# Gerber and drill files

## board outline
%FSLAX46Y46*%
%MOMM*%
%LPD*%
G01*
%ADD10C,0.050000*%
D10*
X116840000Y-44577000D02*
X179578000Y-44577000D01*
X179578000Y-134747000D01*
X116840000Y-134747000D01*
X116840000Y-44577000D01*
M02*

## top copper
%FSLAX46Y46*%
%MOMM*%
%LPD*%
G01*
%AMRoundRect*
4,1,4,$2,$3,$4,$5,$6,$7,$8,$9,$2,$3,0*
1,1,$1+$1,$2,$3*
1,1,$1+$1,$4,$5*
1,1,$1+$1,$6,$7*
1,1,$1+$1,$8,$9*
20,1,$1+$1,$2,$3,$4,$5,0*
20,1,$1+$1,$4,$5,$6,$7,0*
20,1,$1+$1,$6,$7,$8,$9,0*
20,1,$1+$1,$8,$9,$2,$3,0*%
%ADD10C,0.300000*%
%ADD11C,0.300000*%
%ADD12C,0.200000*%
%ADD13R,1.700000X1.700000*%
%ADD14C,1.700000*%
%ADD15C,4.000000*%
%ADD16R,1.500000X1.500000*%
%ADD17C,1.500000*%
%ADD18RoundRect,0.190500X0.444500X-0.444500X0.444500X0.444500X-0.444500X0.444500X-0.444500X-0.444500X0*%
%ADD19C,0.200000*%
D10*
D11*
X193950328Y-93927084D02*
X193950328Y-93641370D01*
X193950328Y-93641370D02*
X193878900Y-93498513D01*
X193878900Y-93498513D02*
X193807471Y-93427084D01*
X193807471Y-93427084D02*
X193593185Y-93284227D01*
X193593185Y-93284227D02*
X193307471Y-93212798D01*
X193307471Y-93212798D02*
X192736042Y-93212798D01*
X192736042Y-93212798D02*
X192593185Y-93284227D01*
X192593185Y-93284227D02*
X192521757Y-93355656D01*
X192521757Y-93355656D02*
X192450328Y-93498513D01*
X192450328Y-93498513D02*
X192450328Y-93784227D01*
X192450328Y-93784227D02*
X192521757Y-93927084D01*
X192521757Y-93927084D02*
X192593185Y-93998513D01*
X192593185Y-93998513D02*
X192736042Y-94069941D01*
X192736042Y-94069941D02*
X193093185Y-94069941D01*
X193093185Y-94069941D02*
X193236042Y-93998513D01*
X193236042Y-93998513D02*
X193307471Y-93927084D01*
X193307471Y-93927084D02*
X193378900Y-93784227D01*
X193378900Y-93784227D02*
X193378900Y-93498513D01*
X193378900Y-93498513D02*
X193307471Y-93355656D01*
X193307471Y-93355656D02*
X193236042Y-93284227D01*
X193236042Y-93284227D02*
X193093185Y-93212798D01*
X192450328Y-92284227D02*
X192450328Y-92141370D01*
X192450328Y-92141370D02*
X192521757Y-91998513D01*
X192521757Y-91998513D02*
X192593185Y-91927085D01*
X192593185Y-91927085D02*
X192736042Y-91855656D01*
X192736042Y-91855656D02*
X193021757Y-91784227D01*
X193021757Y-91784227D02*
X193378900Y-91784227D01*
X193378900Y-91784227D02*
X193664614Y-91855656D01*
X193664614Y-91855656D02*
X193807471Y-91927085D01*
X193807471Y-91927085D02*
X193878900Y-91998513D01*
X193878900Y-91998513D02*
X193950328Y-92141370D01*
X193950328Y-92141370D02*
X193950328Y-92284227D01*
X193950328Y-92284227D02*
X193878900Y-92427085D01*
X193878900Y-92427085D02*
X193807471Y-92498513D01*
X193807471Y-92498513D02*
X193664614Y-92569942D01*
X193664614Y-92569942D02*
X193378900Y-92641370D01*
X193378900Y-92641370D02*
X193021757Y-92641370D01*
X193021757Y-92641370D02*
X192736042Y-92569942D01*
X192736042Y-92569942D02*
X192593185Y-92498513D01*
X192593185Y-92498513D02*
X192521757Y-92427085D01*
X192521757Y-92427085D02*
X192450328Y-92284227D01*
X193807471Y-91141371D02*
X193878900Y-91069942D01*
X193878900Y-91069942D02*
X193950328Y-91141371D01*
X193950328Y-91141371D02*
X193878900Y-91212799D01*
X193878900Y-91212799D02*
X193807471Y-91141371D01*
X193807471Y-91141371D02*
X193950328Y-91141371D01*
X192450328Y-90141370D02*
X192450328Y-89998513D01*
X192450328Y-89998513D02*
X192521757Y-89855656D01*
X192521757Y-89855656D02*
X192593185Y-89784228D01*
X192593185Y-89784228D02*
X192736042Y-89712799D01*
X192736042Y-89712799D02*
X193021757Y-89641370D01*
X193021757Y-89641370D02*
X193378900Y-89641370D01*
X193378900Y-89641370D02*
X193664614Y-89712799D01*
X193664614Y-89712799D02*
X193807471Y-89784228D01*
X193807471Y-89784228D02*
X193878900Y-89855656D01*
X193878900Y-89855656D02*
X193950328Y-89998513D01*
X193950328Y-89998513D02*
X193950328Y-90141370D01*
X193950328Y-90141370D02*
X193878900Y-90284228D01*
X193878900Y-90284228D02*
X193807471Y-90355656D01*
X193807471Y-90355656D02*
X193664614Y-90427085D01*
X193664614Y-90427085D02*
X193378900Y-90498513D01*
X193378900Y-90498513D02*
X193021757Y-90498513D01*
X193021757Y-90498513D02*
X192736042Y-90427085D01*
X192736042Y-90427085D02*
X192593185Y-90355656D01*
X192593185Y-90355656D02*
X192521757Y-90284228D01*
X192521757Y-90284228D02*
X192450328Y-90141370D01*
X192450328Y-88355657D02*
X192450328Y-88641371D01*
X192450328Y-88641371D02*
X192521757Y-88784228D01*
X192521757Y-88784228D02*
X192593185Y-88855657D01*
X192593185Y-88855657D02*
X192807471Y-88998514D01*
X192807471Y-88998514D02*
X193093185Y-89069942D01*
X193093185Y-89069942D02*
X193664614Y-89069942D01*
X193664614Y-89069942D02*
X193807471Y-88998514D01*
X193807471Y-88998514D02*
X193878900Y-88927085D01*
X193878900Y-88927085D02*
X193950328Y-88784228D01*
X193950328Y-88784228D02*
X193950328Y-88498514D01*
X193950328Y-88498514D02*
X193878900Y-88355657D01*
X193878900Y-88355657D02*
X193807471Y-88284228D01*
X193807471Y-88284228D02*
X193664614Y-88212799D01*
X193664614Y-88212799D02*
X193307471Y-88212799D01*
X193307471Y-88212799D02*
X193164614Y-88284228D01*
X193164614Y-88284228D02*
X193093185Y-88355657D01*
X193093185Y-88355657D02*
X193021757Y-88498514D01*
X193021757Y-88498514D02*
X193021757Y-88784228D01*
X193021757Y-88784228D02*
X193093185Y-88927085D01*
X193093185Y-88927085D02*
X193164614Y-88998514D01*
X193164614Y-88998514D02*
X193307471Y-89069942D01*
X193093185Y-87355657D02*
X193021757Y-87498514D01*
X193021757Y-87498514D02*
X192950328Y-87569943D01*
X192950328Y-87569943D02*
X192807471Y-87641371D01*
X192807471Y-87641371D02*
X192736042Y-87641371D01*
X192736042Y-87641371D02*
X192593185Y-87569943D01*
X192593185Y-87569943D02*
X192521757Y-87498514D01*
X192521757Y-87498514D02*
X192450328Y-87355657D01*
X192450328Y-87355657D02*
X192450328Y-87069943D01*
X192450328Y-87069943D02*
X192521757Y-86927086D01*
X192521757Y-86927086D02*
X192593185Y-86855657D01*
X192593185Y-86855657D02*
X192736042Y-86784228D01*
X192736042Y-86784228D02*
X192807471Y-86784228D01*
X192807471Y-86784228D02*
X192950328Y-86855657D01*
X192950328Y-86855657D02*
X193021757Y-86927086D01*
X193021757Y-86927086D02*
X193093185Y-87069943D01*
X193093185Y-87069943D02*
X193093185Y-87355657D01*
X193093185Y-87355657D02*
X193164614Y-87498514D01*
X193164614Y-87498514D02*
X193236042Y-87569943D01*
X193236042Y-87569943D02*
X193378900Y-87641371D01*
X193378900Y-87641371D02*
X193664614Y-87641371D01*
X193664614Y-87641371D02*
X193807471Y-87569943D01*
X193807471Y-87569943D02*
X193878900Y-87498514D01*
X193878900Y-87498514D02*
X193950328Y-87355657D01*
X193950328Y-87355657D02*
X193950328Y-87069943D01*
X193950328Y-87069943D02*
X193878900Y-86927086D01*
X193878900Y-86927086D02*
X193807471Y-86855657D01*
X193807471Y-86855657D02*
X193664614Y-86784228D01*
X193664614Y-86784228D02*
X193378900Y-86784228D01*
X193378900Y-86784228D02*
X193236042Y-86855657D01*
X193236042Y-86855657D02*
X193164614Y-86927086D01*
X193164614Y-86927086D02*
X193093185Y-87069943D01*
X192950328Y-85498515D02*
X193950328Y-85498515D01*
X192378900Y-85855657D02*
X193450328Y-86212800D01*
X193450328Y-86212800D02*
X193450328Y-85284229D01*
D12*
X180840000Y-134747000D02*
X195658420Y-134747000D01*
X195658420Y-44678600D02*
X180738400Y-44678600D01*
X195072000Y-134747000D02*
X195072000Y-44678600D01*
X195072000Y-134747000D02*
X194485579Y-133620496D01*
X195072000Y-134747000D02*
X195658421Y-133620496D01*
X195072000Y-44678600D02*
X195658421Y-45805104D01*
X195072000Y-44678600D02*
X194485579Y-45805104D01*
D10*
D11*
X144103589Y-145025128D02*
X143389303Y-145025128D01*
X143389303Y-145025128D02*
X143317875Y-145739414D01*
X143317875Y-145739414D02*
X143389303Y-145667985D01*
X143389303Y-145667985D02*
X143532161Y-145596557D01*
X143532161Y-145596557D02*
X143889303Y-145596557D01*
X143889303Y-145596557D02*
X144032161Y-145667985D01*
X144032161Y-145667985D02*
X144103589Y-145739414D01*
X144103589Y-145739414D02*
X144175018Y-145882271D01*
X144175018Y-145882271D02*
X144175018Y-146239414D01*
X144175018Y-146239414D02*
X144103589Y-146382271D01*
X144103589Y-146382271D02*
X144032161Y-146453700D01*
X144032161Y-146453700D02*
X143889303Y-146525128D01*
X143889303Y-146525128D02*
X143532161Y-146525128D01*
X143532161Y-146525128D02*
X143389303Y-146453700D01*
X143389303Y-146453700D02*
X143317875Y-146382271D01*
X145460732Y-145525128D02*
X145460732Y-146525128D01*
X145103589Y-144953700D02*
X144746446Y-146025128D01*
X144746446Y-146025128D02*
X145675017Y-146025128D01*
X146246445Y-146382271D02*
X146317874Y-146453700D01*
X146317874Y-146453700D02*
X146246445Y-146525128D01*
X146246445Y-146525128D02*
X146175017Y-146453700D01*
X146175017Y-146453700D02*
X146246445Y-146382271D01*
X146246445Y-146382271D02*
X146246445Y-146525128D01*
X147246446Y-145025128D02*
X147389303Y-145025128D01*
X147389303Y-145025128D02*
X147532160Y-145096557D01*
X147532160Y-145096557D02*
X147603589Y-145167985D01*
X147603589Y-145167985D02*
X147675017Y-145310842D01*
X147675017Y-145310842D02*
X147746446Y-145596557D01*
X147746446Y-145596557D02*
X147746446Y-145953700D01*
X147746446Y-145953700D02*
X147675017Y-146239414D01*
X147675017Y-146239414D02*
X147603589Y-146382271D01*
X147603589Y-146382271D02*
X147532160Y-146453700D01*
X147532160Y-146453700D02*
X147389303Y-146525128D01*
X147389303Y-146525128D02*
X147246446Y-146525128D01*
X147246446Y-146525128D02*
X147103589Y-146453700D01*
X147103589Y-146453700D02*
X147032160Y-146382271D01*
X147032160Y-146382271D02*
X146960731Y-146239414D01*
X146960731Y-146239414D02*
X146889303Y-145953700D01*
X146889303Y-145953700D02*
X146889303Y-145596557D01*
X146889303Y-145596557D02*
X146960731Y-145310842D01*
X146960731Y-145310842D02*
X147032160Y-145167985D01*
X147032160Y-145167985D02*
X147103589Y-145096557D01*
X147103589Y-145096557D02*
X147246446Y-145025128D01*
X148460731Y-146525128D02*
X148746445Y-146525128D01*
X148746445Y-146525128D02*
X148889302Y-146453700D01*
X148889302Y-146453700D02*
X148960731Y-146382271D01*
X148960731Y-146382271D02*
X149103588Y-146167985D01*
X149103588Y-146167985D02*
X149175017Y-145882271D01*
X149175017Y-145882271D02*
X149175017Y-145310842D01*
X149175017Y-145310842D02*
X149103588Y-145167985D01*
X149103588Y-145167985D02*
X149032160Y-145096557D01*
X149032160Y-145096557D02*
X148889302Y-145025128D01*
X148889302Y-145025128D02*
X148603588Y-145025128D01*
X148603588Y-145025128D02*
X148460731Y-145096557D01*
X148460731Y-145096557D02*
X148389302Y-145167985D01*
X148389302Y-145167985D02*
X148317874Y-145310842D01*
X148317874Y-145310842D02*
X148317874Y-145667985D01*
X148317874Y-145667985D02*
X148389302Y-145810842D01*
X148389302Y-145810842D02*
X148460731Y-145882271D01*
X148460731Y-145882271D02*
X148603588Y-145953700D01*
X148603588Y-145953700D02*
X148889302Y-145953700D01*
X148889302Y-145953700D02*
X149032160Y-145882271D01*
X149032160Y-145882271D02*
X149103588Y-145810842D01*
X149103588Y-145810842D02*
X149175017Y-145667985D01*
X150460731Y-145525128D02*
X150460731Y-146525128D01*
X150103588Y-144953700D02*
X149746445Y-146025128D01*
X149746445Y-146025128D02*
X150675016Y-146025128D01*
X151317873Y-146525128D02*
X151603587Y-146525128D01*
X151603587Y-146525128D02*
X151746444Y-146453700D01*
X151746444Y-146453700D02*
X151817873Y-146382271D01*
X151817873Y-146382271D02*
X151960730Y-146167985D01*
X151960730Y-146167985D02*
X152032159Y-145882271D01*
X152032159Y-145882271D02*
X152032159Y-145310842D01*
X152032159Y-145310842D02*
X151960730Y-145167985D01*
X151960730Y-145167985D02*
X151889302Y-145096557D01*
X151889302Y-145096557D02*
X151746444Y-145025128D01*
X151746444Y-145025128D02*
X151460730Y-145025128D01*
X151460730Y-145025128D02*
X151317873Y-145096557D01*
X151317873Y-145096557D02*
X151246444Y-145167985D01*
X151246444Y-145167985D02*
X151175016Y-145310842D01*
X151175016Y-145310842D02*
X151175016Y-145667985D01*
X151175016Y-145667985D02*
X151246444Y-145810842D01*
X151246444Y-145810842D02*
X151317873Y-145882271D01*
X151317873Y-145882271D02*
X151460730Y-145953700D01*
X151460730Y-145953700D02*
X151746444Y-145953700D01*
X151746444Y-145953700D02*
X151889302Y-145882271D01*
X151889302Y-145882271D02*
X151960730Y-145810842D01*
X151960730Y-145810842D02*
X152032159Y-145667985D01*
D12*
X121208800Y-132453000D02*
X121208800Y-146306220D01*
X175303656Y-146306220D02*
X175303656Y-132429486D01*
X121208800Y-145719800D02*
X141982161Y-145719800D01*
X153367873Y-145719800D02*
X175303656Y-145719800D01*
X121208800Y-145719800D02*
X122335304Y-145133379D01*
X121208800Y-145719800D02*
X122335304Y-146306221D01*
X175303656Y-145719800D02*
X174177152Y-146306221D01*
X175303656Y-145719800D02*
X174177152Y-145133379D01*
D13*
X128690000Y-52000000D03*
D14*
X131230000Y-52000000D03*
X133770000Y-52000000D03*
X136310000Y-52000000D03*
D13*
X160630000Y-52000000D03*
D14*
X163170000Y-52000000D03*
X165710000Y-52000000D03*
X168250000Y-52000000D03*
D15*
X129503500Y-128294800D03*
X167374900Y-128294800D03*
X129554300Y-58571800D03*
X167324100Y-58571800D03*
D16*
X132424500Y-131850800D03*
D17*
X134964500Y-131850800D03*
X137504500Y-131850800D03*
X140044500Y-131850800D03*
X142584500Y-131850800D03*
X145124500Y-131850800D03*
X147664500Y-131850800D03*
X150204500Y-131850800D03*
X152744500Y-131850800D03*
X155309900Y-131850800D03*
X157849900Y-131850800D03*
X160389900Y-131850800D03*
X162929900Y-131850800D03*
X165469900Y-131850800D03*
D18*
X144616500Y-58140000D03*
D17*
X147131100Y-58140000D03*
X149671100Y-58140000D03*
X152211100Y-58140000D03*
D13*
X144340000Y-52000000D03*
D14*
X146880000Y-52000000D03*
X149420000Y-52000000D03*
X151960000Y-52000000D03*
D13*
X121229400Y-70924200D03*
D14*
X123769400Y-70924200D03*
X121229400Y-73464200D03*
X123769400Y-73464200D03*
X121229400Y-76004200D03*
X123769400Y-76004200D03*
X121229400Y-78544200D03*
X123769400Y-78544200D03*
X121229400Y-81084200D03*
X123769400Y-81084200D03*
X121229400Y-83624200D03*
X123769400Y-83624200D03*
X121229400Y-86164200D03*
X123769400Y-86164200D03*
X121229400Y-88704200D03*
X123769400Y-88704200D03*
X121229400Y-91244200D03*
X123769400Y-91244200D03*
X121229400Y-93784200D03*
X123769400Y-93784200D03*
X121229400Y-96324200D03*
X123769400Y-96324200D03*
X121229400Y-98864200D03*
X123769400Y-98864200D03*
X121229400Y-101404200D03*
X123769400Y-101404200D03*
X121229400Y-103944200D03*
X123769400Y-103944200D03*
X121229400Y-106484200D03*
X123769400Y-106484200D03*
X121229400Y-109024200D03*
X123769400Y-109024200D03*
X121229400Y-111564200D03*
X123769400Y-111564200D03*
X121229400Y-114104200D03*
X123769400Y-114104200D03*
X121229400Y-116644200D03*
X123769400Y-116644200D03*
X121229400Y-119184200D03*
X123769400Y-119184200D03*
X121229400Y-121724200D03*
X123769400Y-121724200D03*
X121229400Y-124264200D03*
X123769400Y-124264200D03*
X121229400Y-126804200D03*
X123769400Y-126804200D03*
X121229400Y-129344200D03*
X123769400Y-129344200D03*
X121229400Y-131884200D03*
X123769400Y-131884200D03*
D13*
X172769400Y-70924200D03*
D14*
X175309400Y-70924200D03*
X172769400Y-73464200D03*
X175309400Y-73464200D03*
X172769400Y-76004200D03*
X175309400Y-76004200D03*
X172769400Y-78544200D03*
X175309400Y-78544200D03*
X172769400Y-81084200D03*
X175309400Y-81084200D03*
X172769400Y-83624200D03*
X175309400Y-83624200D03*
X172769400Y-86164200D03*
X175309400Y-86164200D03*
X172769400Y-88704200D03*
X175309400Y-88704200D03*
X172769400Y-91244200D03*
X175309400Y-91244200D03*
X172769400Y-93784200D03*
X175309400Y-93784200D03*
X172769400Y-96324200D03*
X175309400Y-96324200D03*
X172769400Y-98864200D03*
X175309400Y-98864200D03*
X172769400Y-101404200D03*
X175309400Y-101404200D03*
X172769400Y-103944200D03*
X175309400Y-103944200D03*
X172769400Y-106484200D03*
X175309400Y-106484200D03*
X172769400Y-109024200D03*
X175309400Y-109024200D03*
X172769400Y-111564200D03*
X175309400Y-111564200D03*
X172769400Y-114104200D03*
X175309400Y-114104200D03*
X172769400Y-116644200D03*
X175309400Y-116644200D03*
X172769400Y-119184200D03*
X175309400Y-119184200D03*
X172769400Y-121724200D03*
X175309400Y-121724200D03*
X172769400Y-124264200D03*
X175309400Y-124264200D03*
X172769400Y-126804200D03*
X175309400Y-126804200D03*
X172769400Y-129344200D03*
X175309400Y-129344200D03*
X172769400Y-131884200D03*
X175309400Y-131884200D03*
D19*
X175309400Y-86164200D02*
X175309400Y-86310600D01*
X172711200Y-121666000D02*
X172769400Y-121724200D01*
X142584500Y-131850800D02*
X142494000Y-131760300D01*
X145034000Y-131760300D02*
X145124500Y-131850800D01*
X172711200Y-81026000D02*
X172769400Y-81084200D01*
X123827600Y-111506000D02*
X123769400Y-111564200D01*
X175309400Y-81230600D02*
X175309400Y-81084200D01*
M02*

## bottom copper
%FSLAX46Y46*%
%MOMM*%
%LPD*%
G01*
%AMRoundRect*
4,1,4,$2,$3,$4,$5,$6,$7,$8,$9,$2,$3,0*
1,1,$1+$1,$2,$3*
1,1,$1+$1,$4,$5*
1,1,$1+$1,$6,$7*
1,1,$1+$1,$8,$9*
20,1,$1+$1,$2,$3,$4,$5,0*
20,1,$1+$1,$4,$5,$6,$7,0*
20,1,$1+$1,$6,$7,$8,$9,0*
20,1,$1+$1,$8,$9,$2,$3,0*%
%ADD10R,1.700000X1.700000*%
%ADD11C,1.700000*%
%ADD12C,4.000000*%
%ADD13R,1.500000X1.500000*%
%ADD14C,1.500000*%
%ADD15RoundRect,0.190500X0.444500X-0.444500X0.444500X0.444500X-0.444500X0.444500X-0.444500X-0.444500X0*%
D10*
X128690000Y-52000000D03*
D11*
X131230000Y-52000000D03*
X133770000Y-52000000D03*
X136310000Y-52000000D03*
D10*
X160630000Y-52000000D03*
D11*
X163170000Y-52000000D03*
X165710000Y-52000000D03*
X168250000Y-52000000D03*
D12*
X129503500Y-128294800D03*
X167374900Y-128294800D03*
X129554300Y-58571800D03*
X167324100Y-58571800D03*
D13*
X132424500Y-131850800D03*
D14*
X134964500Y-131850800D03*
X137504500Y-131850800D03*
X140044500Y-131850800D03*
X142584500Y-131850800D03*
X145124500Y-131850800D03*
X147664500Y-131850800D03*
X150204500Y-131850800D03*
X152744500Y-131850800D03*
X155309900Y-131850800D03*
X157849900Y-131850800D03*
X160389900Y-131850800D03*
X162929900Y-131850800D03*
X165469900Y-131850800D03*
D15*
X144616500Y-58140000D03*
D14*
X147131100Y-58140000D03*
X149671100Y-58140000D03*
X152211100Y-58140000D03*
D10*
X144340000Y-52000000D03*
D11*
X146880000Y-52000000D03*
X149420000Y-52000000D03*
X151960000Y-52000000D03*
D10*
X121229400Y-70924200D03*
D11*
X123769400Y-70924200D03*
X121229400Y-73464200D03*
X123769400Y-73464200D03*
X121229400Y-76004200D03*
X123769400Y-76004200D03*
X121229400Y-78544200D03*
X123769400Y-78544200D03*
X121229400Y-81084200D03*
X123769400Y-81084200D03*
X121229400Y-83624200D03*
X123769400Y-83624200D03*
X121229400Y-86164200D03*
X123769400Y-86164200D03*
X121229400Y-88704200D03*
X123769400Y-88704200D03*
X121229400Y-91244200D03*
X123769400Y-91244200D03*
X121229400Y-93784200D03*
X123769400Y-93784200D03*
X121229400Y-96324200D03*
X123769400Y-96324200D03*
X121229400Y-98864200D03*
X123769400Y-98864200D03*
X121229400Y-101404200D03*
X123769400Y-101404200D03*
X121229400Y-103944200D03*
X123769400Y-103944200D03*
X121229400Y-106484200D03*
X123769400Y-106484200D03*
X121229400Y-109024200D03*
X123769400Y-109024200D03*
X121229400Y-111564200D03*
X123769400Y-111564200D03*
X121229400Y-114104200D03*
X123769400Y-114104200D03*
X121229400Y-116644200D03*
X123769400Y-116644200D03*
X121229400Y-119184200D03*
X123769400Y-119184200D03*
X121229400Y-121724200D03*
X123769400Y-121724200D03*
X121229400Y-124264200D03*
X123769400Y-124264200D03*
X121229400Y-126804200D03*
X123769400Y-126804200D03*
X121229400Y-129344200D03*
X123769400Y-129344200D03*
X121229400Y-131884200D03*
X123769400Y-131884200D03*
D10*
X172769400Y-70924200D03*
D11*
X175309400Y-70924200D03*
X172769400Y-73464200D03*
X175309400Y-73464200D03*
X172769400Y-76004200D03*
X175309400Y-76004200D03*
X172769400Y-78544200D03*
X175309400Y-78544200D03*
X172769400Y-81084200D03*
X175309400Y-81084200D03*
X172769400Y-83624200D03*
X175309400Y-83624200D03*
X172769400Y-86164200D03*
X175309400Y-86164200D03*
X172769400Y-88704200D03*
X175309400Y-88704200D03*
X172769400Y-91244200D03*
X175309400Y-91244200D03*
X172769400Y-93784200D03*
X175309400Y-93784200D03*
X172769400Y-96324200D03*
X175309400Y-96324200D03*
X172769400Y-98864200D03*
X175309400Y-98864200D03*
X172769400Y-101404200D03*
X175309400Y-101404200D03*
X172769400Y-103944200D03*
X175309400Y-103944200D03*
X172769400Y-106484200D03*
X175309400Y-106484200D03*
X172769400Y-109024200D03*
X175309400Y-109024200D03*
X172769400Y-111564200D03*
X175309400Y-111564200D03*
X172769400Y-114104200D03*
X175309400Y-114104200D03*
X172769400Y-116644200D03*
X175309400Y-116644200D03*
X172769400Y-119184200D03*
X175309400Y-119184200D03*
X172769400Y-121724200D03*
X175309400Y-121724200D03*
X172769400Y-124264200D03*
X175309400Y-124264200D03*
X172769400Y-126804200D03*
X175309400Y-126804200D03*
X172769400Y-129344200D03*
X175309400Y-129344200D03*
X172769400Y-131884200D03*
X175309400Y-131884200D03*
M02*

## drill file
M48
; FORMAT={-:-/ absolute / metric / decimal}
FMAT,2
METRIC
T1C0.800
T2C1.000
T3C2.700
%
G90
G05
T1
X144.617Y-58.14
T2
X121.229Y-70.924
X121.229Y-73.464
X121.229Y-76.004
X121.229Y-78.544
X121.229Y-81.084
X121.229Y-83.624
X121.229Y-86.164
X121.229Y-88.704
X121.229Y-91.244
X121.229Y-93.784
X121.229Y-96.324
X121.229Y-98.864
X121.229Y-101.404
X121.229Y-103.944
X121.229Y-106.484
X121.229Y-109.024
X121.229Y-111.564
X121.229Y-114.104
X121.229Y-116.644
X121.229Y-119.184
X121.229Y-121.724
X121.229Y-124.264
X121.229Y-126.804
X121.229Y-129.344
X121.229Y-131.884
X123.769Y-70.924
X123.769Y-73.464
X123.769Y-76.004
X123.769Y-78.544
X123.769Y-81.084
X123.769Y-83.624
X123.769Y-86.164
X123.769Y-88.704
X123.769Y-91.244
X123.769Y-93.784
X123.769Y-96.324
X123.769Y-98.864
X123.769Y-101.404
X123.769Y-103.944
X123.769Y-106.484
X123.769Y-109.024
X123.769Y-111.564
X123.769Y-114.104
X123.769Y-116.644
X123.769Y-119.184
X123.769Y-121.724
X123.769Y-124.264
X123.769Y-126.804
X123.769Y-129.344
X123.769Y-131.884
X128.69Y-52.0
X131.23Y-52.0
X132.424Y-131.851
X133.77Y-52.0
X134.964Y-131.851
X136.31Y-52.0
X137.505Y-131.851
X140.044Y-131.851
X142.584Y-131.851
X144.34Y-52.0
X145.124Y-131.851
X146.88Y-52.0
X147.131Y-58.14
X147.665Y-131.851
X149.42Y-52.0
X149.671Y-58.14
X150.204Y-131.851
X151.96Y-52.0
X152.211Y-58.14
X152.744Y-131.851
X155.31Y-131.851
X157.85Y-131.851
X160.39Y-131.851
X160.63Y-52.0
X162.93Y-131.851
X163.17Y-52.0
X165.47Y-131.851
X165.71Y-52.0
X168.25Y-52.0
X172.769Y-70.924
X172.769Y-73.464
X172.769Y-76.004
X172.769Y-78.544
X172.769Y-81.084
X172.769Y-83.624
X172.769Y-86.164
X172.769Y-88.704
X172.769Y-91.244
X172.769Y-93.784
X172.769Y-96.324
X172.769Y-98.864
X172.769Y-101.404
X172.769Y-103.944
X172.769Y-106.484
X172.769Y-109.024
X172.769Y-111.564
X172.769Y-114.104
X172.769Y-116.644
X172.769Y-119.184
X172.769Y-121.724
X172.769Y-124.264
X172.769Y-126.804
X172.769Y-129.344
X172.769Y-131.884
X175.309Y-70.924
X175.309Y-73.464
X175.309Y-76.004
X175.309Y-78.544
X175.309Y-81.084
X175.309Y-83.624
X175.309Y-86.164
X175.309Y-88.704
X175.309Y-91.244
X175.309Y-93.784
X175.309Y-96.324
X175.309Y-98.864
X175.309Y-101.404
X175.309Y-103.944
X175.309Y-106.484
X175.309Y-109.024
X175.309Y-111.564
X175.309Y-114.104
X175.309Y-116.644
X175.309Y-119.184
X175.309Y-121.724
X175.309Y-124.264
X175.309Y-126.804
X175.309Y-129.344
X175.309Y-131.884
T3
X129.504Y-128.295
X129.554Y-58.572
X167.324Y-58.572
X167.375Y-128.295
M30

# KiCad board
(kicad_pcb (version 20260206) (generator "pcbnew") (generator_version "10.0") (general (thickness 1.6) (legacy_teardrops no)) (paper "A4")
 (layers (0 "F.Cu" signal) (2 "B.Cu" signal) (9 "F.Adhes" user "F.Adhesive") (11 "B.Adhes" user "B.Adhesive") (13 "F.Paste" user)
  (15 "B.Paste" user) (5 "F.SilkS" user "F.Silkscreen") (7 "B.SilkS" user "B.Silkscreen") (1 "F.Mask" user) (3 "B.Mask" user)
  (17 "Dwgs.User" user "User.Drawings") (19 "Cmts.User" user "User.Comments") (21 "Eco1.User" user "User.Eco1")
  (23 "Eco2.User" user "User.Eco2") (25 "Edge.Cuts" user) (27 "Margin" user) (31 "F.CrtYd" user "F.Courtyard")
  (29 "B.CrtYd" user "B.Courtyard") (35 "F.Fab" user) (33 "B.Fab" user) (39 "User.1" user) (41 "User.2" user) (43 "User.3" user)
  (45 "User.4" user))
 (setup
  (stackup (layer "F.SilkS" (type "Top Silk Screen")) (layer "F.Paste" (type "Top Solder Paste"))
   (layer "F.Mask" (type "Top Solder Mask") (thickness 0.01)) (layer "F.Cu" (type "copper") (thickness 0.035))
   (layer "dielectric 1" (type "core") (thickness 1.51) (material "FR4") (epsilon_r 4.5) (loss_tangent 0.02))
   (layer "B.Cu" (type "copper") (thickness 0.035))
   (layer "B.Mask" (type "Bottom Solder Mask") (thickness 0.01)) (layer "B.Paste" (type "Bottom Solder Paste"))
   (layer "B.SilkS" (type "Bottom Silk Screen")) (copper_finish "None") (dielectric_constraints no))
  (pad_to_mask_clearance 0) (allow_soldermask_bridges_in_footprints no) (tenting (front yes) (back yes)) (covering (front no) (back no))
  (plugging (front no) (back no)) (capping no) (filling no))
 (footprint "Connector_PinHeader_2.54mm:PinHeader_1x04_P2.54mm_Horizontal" (layer "F.Cu") (at 128.69 52 90)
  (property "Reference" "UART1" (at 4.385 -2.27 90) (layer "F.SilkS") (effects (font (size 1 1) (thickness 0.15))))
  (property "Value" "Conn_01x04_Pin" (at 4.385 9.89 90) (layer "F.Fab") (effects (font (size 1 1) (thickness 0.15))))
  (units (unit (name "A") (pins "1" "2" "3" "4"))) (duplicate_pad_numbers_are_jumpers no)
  (pad "1" thru_hole rect (at 0 0 90) (size 1.7 1.7) (drill 1) (layers "*.Cu" "*.Mask") (remove_unused_layers no) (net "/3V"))
  (pad "2" thru_hole circle (at 0 2.54 90) (size 1.7 1.7) (drill 1) (layers "*.Cu" "*.Mask") (remove_unused_layers no) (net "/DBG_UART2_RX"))
  (pad "3" thru_hole circle (at 0 5.08 90) (size 1.7 1.7) (drill 1) (layers "*.Cu" "*.Mask") (remove_unused_layers no) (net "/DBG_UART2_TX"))
  (pad "4" thru_hole circle (at 0 7.62 90) (size 1.7 1.7) (drill 1) (layers "*.Cu" "*.Mask") (remove_unused_layers no) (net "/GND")))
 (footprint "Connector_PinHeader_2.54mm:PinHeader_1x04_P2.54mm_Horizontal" (layer "F.Cu") (at 160.63 52 90)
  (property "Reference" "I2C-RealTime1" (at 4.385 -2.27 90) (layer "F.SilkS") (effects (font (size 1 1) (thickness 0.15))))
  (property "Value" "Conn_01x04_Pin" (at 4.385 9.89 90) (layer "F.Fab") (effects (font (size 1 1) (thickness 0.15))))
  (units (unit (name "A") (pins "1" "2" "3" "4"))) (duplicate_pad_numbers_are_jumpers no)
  (pad "1" thru_hole rect (at 0 0 90) (size 1.7 1.7) (drill 1) (layers "*.Cu" "*.Mask") (remove_unused_layers no) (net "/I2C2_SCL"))
  (pad "2" thru_hole circle (at 0 2.54 90) (size 1.7 1.7) (drill 1) (layers "*.Cu" "*.Mask") (remove_unused_layers no) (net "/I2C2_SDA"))
  (pad "3" thru_hole circle (at 0 5.08 90) (size 1.7 1.7) (drill 1) (layers "*.Cu" "*.Mask") (remove_unused_layers no) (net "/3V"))
  (pad "4" thru_hole circle (at 0 7.62 90) (size 1.7 1.7) (drill 1) (layers "*.Cu" "*.Mask") (remove_unused_layers no) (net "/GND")))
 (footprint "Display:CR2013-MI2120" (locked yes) (layer "F.Cu") (at 137.5045 131.8508 90)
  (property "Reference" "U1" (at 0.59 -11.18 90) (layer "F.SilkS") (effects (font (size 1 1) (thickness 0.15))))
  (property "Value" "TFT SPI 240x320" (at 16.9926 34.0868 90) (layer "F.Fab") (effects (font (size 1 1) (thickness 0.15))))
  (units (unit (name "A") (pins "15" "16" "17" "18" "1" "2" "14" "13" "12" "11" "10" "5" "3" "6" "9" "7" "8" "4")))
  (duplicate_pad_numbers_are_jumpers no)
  (pad "" thru_hole circle (at 3.556 -8.001 90) (size 4 4) (drill 2.7) (layers "*.Cu" "*.Mask") (remove_unused_layers no))
  (pad "" thru_hole circle (at 3.556 29.8704 90) (size 4 4) (drill 2.7) (layers "*.Cu" "*.Mask") (remove_unused_layers no))
  (pad "" thru_hole circle (at 73.279 -7.9502 90) (size 4 4) (drill 2.7) (layers "*.Cu" "*.Mask") (remove_unused_layers no))
  (pad "" thru_hole circle (at 73.279 29.8196 90) (size 4 4) (drill 2.7) (layers "*.Cu" "*.Mask") (remove_unused_layers no))
  (pad "1" thru_hole rect (at 0 -5.08 90) (size 1.5 1.5) (drill 1) (layers "*.Cu" "*.Mask") (remove_unused_layers no) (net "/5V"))
  (pad "2" thru_hole circle (at 0 -2.54 90) (size 1.5 1.5) (drill 1) (layers "*.Cu" "*.Mask") (remove_unused_layers no) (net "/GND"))
  (pad "3" thru_hole circle (at 0 0 90) (size 1.5 1.5) (drill 1) (layers "*.Cu" "*.Mask") (remove_unused_layers no) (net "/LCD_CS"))
  (pad "4" thru_hole circle (at 0 2.54 90) (size 1.5 1.5) (drill 1) (layers "*.Cu" "*.Mask") (remove_unused_layers no) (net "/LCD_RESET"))
  (pad "5" thru_hole circle (at 0 5.08 90) (size 1.5 1.5) (drill 1) (layers "*.Cu" "*.Mask") (remove_unused_layers no) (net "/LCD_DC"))
  (pad "6" thru_hole circle (at 0 7.62 90) (size 1.5 1.5) (drill 1) (layers "*.Cu" "*.Mask") (remove_unused_layers no) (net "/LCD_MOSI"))
  (pad "7" thru_hole circle (at 0 10.16 90) (size 1.5 1.5) (drill 1) (layers "*.Cu" "*.Mask") (remove_unused_layers no) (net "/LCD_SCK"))
  (pad "8" thru_hole circle (at 0 12.7 90) (size 1.5 1.5) (drill 1) (layers "*.Cu" "*.Mask") (remove_unused_layers no) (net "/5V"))
  (pad "9" thru_hole circle (at 0 15.24 90) (size 1.5 1.5) (drill 1) (layers "*.Cu" "*.Mask") (remove_unused_layers no) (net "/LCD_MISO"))
  (pad "10" thru_hole circle (at 0 17.8054 90) (size 1.5 1.5) (drill 1) (layers "*.Cu" "*.Mask") (remove_unused_layers no)
   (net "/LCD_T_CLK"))
  (pad "11" thru_hole circle (at 0 20.3454 90) (size 1.5 1.5) (drill 1) (layers "*.Cu" "*.Mask") (remove_unused_layers no) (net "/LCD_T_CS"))
  (pad "12" thru_hole circle (at 0 22.8854 90) (size 1.5 1.5) (drill 1) (layers "*.Cu" "*.Mask") (remove_unused_layers no)
   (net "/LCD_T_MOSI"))
  (pad "13" thru_hole circle (at 0 25.4254 90) (size 1.5 1.5) (drill 1) (layers "*.Cu" "*.Mask") (remove_unused_layers no)
   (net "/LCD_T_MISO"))
  (pad "14" thru_hole circle (at 0 27.9654 90) (size 1.5 1.5) (drill 1) (layers "*.Cu" "*.Mask") (remove_unused_layers no)
   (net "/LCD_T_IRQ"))
  (pad "15" thru_hole roundrect (at 73.7108 7.112 90) (size 1.27 1.27) (drill 0.8) (layers "*.Cu" "*.Mask") (remove_unused_layers no)
   (roundrect_rratio 0.15) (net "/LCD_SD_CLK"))
  (pad "16" thru_hole circle (at 73.7108 9.6266 90) (size 1.5 1.5) (drill 1) (layers "*.Cu" "*.Mask") (remove_unused_layers no)
   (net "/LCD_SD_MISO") (thermal_bridge_angle 90))
  (pad "17" thru_hole circle (at 73.7108 12.1666 90) (size 1.5 1.5) (drill 1) (layers "*.Cu" "*.Mask") (remove_unused_layers no)
   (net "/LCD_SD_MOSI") (thermal_bridge_angle 90))
  (pad "18" thru_hole circle (at 73.7108 14.7066 90) (size 1.5 1.5) (drill 1) (layers "*.Cu" "*.Mask") (remove_unused_layers no)
   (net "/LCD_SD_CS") (thermal_bridge_angle 90)))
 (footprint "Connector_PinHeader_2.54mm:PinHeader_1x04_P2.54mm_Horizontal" (layer "F.Cu") (at 144.34 52 90)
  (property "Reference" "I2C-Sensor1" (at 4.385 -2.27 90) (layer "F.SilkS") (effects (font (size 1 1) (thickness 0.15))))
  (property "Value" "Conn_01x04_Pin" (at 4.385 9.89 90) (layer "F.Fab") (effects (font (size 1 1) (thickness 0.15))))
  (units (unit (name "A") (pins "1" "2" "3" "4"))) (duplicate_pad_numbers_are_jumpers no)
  (pad "1" thru_hole rect (at 0 0 90) (size 1.7 1.7) (drill 1) (layers "*.Cu" "*.Mask") (remove_unused_layers no) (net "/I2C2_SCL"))
  (pad "2" thru_hole circle (at 0 2.54 90) (size 1.7 1.7) (drill 1) (layers "*.Cu" "*.Mask") (remove_unused_layers no) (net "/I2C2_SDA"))
  (pad "3" thru_hole circle (at 0 5.08 90) (size 1.7 1.7) (drill 1) (layers "*.Cu" "*.Mask") (remove_unused_layers no) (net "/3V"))
  (pad "4" thru_hole circle (at 0 7.62 90) (size 1.7 1.7) (drill 1) (layers "*.Cu" "*.Mask") (remove_unused_layers no) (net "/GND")))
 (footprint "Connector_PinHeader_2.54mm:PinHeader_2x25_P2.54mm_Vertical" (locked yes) (layer "F.Cu") (at 121.2294 70.9242)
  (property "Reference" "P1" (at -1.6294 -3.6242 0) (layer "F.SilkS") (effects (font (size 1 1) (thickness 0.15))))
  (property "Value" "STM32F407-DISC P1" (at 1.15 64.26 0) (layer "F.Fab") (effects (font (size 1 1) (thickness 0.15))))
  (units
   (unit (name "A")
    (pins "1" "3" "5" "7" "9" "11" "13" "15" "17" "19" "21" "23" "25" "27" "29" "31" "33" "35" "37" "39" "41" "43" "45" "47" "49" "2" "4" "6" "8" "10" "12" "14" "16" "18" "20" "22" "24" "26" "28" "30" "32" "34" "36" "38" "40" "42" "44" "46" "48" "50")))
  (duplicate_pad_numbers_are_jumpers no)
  (pad "1" thru_hole rect (at 0 0) (size 1.7 1.7) (drill 1) (layers "*.Cu" "*.Mask") (remove_unused_layers no) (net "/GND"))
  (pad "2" thru_hole circle (at 2.54 0) (size 1.7 1.7) (drill 1) (layers "*.Cu" "*.Mask") (remove_unused_layers no) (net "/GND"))
  (pad "3" thru_hole circle (at 0 2.54) (size 1.7 1.7) (drill 1) (layers "*.Cu" "*.Mask") (remove_unused_layers no) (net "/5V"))
  (pad "4" thru_hole circle (at 2.54 2.54) (size 1.7 1.7) (drill 1) (layers "*.Cu" "*.Mask") (remove_unused_layers no) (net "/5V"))
  (pad "5" thru_hole circle (at 0 5.08) (size 1.7 1.7) (drill 1) (layers "*.Cu" "*.Mask") (remove_unused_layers no) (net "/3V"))
  (pad "6" thru_hole circle (at 2.54 5.08) (size 1.7 1.7) (drill 1) (layers "*.Cu" "*.Mask") (remove_unused_layers no) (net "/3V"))
  (pad "7" thru_hole circle (at 0 7.62) (size 1.7 1.7) (drill 1) (layers "*.Cu" "*.Mask") (remove_unused_layers no) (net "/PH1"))
  (pad "8" thru_hole circle (at 2.54 7.62) (size 1.7 1.7) (drill 1) (layers "*.Cu" "*.Mask") (remove_unused_layers no) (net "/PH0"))
  (pad "9" thru_hole circle (at 0 10.16) (size 1.7 1.7) (drill 1) (layers "*.Cu" "*.Mask") (remove_unused_layers no) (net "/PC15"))
  (pad "10" thru_hole circle (at 2.54 10.16) (size 1.7 1.7) (drill 1) (layers "*.Cu" "*.Mask") (remove_unused_layers no) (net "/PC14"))
  (pad "11" thru_hole circle (at 0 12.7) (size 1.7 1.7) (drill 1) (layers "*.Cu" "*.Mask") (remove_unused_layers no) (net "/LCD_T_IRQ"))
  (pad "12" thru_hole circle (at 2.54 12.7) (size 1.7 1.7) (drill 1) (layers "*.Cu" "*.Mask") (remove_unused_layers no) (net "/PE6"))
  (pad "13" thru_hole circle (at 0 15.24) (size 1.7 1.7) (drill 1) (layers "*.Cu" "*.Mask") (remove_unused_layers no) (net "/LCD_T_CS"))
  (pad "14" thru_hole circle (at 2.54 15.24) (size 1.7 1.7) (drill 1) (layers "*.Cu" "*.Mask") (remove_unused_layers no) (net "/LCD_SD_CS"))
  (pad "15" thru_hole circle (at 0 17.78) (size 1.7 1.7) (drill 1) (layers "*.Cu" "*.Mask") (remove_unused_layers no) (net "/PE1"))
  (pad "16" thru_hole circle (at 2.54 17.78) (size 1.7 1.7) (drill 1) (layers "*.Cu" "*.Mask") (remove_unused_layers no) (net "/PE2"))
  (pad "17" thru_hole circle (at 0 20.32) (size 1.7 1.7) (drill 1) (layers "*.Cu" "*.Mask") (remove_unused_layers no) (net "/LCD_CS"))
  (pad "18" thru_hole circle (at 2.54 20.32) (size 1.7 1.7) (drill 1) (layers "*.Cu" "*.Mask") (remove_unused_layers no) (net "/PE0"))
  (pad "19" thru_hole circle (at 0 22.86) (size 1.7 1.7) (drill 1) (layers "*.Cu" "*.Mask") (remove_unused_layers no) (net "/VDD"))
  (pad "20" thru_hole circle (at 2.54 22.86) (size 1.7 1.7) (drill 1) (layers "*.Cu" "*.Mask") (remove_unused_layers no) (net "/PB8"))
  (pad "21" thru_hole circle (at 0 25.4) (size 1.7 1.7) (drill 1) (layers "*.Cu" "*.Mask") (remove_unused_layers no) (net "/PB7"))
  (pad "22" thru_hole circle (at 2.54 25.4) (size 1.7 1.7) (drill 1) (layers "*.Cu" "*.Mask") (remove_unused_layers no) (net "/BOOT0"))
  (pad "23" thru_hole circle (at 0 27.94) (size 1.7 1.7) (drill 1) (layers "*.Cu" "*.Mask") (remove_unused_layers no) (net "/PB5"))
  (pad "24" thru_hole circle (at 2.54 27.94) (size 1.7 1.7) (drill 1) (layers "*.Cu" "*.Mask") (remove_unused_layers no) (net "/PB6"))
  (pad "25" thru_hole circle (at 0 30.48) (size 1.7 1.7) (drill 1) (layers "*.Cu" "*.Mask") (remove_unused_layers no) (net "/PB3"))
  (pad "26" thru_hole circle (at 2.54 30.48) (size 1.7 1.7) (drill 1) (layers "*.Cu" "*.Mask") (remove_unused_layers no) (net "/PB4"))
  (pad "27" thru_hole circle (at 0 33.02) (size 1.7 1.7) (drill 1) (layers "*.Cu" "*.Mask") (remove_unused_layers no) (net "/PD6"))
  (pad "28" thru_hole circle (at 2.54 33.02) (size 1.7 1.7) (drill 1) (layers "*.Cu" "*.Mask") (remove_unused_layers no) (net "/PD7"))
  (pad "29" thru_hole circle (at 0 35.56) (size 1.7 1.7) (drill 1) (layers "*.Cu" "*.Mask") (remove_unused_layers no) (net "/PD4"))
  (pad "30" thru_hole circle (at 2.54 35.56) (size 1.7 1.7) (drill 1) (layers "*.Cu" "*.Mask") (remove_unused_layers no) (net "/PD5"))
  (pad "31" thru_hole circle (at 0 38.1) (size 1.7 1.7) (drill 1) (layers "*.Cu" "*.Mask") (remove_unused_layers no) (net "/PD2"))
  (pad "32" thru_hole circle (at 2.54 38.1) (size 1.7 1.7) (drill 1) (layers "*.Cu" "*.Mask") (remove_unused_layers no) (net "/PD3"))
  (pad "33" thru_hole circle (at 0 40.64) (size 1.7 1.7) (drill 1) (layers "*.Cu" "*.Mask") (remove_unused_layers no) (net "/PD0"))
  (pad "34" thru_hole circle (at 2.54 40.64) (size 1.7 1.7) (drill 1) (layers "*.Cu" "*.Mask") (remove_unused_layers no) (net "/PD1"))
  (pad "35" thru_hole circle (at 0 43.18) (size 1.7 1.7) (drill 1) (layers "*.Cu" "*.Mask") (remove_unused_layers no) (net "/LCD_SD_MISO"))
  (pad "36" thru_hole circle (at 2.54 43.18) (size 1.7 1.7) (drill 1) (layers "*.Cu" "*.Mask") (remove_unused_layers no)
   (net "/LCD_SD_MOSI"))
  (pad "37" thru_hole circle (at 0 45.72) (size 1.7 1.7) (drill 1) (layers "*.Cu" "*.Mask") (remove_unused_layers no) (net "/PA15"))
  (pad "38" thru_hole circle (at 2.54 45.72) (size 1.7 1.7) (drill 1) (layers "*.Cu" "*.Mask") (remove_unused_layers no) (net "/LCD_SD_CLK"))
  (pad "39" thru_hole circle (at 0 48.26) (size 1.7 1.7) (drill 1) (layers "*.Cu" "*.Mask") (remove_unused_layers no) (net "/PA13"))
  (pad "40" thru_hole circle (at 2.54 48.26) (size 1.7 1.7) (drill 1) (layers "*.Cu" "*.Mask") (remove_unused_layers no) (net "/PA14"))
  (pad "41" thru_hole circle (at 0 50.8) (size 1.7 1.7) (drill 1) (layers "*.Cu" "*.Mask") (remove_unused_layers no) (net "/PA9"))
  (pad "42" thru_hole circle (at 2.54 50.8) (size 1.7 1.7) (drill 1) (layers "*.Cu" "*.Mask") (remove_unused_layers no) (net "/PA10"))
  (pad "43" thru_hole circle (at 0 53.34) (size 1.7 1.7) (drill 1) (layers "*.Cu" "*.Mask") (remove_unused_layers no) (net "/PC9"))
  (pad "44" thru_hole circle (at 2.54 53.34) (size 1.7 1.7) (drill 1) (layers "*.Cu" "*.Mask") (remove_unused_layers no) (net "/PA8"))
  (pad "45" thru_hole circle (at 0 55.88) (size 1.7 1.7) (drill 1) (layers "*.Cu" "*.Mask") (remove_unused_layers no) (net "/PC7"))
  (pad "46" thru_hole circle (at 2.54 55.88) (size 1.7 1.7) (drill 1) (layers "*.Cu" "*.Mask") (remove_unused_layers no) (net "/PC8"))
  (pad "47" thru_hole circle (at 0 58.42) (size 1.7 1.7) (drill 1) (layers "*.Cu" "*.Mask") (remove_unused_layers no) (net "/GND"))
  (pad "48" thru_hole circle (at 2.54 58.42) (size 1.7 1.7) (drill 1) (layers "*.Cu" "*.Mask") (remove_unused_layers no) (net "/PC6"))
  (pad "49" thru_hole circle (at 0 60.96) (size 1.7 1.7) (drill 1) (layers "*.Cu" "*.Mask") (remove_unused_layers no) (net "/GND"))
  (pad "50" thru_hole circle (at 2.54 60.96) (size 1.7 1.7) (drill 1) (layers "*.Cu" "*.Mask") (remove_unused_layers no) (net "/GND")))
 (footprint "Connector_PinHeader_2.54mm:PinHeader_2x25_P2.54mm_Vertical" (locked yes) (layer "F.Cu") (at 172.7694 70.9242)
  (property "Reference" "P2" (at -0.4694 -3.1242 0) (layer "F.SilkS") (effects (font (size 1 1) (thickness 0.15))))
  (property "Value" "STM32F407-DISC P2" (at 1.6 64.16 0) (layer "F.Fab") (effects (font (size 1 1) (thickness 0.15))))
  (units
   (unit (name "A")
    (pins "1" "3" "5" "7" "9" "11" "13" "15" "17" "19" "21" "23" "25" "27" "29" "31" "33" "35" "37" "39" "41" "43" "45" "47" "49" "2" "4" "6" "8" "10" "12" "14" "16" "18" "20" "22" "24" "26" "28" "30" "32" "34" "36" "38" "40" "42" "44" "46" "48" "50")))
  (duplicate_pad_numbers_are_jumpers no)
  (pad "1" thru_hole rect (at 0 0) (size 1.7 1.7) (drill 1) (layers "*.Cu" "*.Mask") (remove_unused_layers no) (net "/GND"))
  (pad "2" thru_hole circle (at 2.54 0) (size 1.7 1.7) (drill 1) (layers "*.Cu" "*.Mask") (remove_unused_layers no) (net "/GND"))
  (pad "3" thru_hole circle (at 0 2.54) (size 1.7 1.7) (drill 1) (layers "*.Cu" "*.Mask") (remove_unused_layers no) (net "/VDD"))
  (pad "4" thru_hole circle (at 2.54 2.54) (size 1.7 1.7) (drill 1) (layers "*.Cu" "*.Mask") (remove_unused_layers no) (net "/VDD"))
  (pad "5" thru_hole circle (at 0 5.08) (size 1.7 1.7) (drill 1) (layers "*.Cu" "*.Mask") (remove_unused_layers no) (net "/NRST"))
  (pad "6" thru_hole circle (at 2.54 5.08) (size 1.7 1.7) (drill 1) (layers "*.Cu" "*.Mask") (remove_unused_layers no) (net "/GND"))
  (pad "7" thru_hole circle (at 0 7.62) (size 1.7 1.7) (drill 1) (layers "*.Cu" "*.Mask") (remove_unused_layers no) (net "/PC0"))
  (pad "8" thru_hole circle (at 2.54 7.62) (size 1.7 1.7) (drill 1) (layers "*.Cu" "*.Mask") (remove_unused_layers no) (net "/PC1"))
  (pad "9" thru_hole circle (at 0 10.16) (size 1.7 1.7) (drill 1) (layers "*.Cu" "*.Mask") (remove_unused_layers no) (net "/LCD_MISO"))
  (pad "10" thru_hole circle (at 2.54 10.16) (size 1.7 1.7) (drill 1) (layers "*.Cu" "*.Mask") (remove_unused_layers no) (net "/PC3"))
  (pad "11" thru_hole circle (at 0 12.7) (size 1.7 1.7) (drill 1) (layers "*.Cu" "*.Mask") (remove_unused_layers no) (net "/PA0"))
  (pad "12" thru_hole circle (at 2.54 12.7) (size 1.7 1.7) (drill 1) (layers "*.Cu" "*.Mask") (remove_unused_layers no) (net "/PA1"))
  (pad "13" thru_hole circle (at 0 15.24) (size 1.7 1.7) (drill 1) (layers "*.Cu" "*.Mask") (remove_unused_layers no) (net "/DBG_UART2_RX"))
  (pad "14" thru_hole circle (at 2.54 15.24) (size 1.7 1.7) (drill 1) (layers "*.Cu" "*.Mask") (remove_unused_layers no)
   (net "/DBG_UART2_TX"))
  (pad "15" thru_hole circle (at 0 17.78) (size 1.7 1.7) (drill 1) (layers "*.Cu" "*.Mask") (remove_unused_layers no) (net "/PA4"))
  (pad "16" thru_hole circle (at 2.54 17.78) (size 1.7 1.7) (drill 1) (layers "*.Cu" "*.Mask") (remove_unused_layers no) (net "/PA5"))
  (pad "17" thru_hole circle (at 0 20.32) (size 1.7 1.7) (drill 1) (layers "*.Cu" "*.Mask") (remove_unused_layers no) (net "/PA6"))
  (pad "18" thru_hole circle (at 2.54 20.32) (size 1.7 1.7) (drill 1) (layers "*.Cu" "*.Mask") (remove_unused_layers no) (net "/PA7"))
  (pad "19" thru_hole circle (at 0 22.86) (size 1.7 1.7) (drill 1) (layers "*.Cu" "*.Mask") (remove_unused_layers no) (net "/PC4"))
  (pad "20" thru_hole circle (at 2.54 22.86) (size 1.7 1.7) (drill 1) (layers "*.Cu" "*.Mask") (remove_unused_layers no) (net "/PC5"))
  (pad "21" thru_hole circle (at 0 25.4) (size 1.7 1.7) (drill 1) (layers "*.Cu" "*.Mask") (remove_unused_layers no) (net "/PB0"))
  (pad "22" thru_hole circle (at 2.54 25.4) (size 1.7 1.7) (drill 1) (layers "*.Cu" "*.Mask") (remove_unused_layers no) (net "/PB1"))
  (pad "23" thru_hole circle (at 0 27.94) (size 1.7 1.7) (drill 1) (layers "*.Cu" "*.Mask") (remove_unused_layers no) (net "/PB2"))
  (pad "24" thru_hole circle (at 2.54 27.94) (size 1.7 1.7) (drill 1) (layers "*.Cu" "*.Mask") (remove_unused_layers no) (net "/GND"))
  (pad "25" thru_hole circle (at 0 30.48) (size 1.7 1.7) (drill 1) (layers "*.Cu" "*.Mask") (remove_unused_layers no) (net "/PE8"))
  (pad "26" thru_hole circle (at 2.54 30.48) (size 1.7 1.7) (drill 1) (layers "*.Cu" "*.Mask") (remove_unused_layers no) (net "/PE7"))
  (pad "27" thru_hole circle (at 0 33.02) (size 1.7 1.7) (drill 1) (layers "*.Cu" "*.Mask") (remove_unused_layers no) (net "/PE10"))
  (pad "28" thru_hole circle (at 2.54 33.02) (size 1.7 1.7) (drill 1) (layers "*.Cu" "*.Mask") (remove_unused_layers no) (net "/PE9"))
  (pad "29" thru_hole circle (at 0 35.56) (size 1.7 1.7) (drill 1) (layers "*.Cu" "*.Mask") (remove_unused_layers no) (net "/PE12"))
  (pad "30" thru_hole circle (at 2.54 35.56) (size 1.7 1.7) (drill 1) (layers "*.Cu" "*.Mask") (remove_unused_layers no) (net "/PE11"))
  (pad "31" thru_hole circle (at 0 38.1) (size 1.7 1.7) (drill 1) (layers "*.Cu" "*.Mask") (remove_unused_layers no) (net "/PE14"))
  (pad "32" thru_hole circle (at 2.54 38.1) (size 1.7 1.7) (drill 1) (layers "*.Cu" "*.Mask") (remove_unused_layers no) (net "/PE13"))
  (pad "33" thru_hole circle (at 0 40.64) (size 1.7 1.7) (drill 1) (layers "*.Cu" "*.Mask") (remove_unused_layers no) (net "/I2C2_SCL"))
  (pad "34" thru_hole circle (at 2.54 40.64) (size 1.7 1.7) (drill 1) (layers "*.Cu" "*.Mask") (remove_unused_layers no) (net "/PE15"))
  (pad "35" thru_hole circle (at 0 43.18) (size 1.7 1.7) (drill 1) (layers "*.Cu" "*.Mask") (remove_unused_layers no) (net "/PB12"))
  (pad "36" thru_hole circle (at 2.54 43.18) (size 1.7 1.7) (drill 1) (layers "*.Cu" "*.Mask") (remove_unused_layers no) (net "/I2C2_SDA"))
  (pad "37" thru_hole circle (at 0 45.72) (size 1.7 1.7) (drill 1) (layers "*.Cu" "*.Mask") (remove_unused_layers no) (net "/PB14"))
  (pad "38" thru_hole circle (at 2.54 45.72) (size 1.7 1.7) (drill 1) (layers "*.Cu" "*.Mask") (remove_unused_layers no) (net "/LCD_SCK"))
  (pad "39" thru_hole circle (at 0 48.26) (size 1.7 1.7) (drill 1) (layers "*.Cu" "*.Mask") (remove_unused_layers no) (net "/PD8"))
  (pad "40" thru_hole circle (at 2.54 48.26) (size 1.7 1.7) (drill 1) (layers "*.Cu" "*.Mask") (remove_unused_layers no) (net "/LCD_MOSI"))
  (pad "41" thru_hole circle (at 0 50.8) (size 1.7 1.7) (drill 1) (layers "*.Cu" "*.Mask") (remove_unused_layers no) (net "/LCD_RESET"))
  (pad "42" thru_hole circle (at 2.54 50.8) (size 1.7 1.7) (drill 1) (layers "*.Cu" "*.Mask") (remove_unused_layers no) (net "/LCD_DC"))
  (pad "43" thru_hole circle (at 0 53.34) (size 1.7 1.7) (drill 1) (layers "*.Cu" "*.Mask") (remove_unused_layers no) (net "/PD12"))
  (pad "44" thru_hole circle (at 2.54 53.34) (size 1.7 1.7) (drill 1) (layers "*.Cu" "*.Mask") (remove_unused_layers no) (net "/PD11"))
  (pad "45" thru_hole circle (at 0 55.88) (size 1.7 1.7) (drill 1) (layers "*.Cu" "*.Mask") (remove_unused_layers no) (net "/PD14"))
  (pad "46" thru_hole circle (at 2.54 55.88) (size 1.7 1.7) (drill 1) (layers "*.Cu" "*.Mask") (remove_unused_layers no) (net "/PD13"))
  (pad "47" thru_hole circle (at 0 58.42) (size 1.7 1.7) (drill 1) (layers "*.Cu" "*.Mask") (remove_unused_layers no) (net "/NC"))
  (pad "48" thru_hole circle (at 2.54 58.42) (size 1.7 1.7) (drill 1) (layers "*.Cu" "*.Mask") (remove_unused_layers no) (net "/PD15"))
  (pad "49" thru_hole circle (at 0 60.96) (size 1.7 1.7) (drill 1) (layers "*.Cu" "*.Mask") (remove_unused_layers no) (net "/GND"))
  (pad "50" thru_hole circle (at 2.54 60.96) (size 1.7 1.7) (drill 1) (layers "*.Cu" "*.Mask") (remove_unused_layers no) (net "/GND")))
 (gr_rect (start 116.84 44.577) (end 179.578 134.747) (stroke (width 0.05) (type default)) (fill no) (layer "Edge.Cuts"))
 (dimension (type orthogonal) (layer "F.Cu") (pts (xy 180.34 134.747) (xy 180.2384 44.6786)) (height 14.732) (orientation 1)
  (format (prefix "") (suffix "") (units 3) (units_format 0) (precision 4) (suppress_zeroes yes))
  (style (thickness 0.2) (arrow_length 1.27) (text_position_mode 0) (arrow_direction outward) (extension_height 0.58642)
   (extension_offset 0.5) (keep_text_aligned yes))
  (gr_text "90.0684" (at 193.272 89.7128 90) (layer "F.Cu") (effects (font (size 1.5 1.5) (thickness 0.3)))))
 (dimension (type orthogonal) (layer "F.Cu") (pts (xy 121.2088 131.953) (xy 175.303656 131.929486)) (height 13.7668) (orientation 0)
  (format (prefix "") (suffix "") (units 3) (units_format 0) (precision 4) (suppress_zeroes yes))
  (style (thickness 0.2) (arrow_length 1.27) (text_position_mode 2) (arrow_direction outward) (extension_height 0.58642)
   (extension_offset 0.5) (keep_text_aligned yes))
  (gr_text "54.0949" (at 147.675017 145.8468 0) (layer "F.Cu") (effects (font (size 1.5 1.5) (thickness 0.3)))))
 (segment (start 175.3094 86.1642) (end 175.3094 86.3106) (width 0.2) (layer "F.Cu") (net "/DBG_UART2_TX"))
 (segment (start 172.7112 121.666) (end 172.7694 121.7242) (width 0.2) (layer "F.Cu") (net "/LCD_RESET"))
 (segment (start 142.5845 131.8508) (end 142.494 131.7603) (width 0.2) (layer "F.Cu") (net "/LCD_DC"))
 (segment (start 145.034 131.7603) (end 145.1245 131.8508) (width 0.2) (layer "F.Cu") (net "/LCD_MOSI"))
 (segment (start 172.7112 81.026) (end 172.7694 81.0842) (width 0.2) (layer "F.Cu") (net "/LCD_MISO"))
 (segment (start 123.8276 111.506) (end 123.7694 111.5642) (width 0.2) (layer "F.Cu") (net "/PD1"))
 (segment (start 175.3094 81.2306) (end 175.3094 81.0842) (width 0.2) (layer "F.Cu") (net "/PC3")))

